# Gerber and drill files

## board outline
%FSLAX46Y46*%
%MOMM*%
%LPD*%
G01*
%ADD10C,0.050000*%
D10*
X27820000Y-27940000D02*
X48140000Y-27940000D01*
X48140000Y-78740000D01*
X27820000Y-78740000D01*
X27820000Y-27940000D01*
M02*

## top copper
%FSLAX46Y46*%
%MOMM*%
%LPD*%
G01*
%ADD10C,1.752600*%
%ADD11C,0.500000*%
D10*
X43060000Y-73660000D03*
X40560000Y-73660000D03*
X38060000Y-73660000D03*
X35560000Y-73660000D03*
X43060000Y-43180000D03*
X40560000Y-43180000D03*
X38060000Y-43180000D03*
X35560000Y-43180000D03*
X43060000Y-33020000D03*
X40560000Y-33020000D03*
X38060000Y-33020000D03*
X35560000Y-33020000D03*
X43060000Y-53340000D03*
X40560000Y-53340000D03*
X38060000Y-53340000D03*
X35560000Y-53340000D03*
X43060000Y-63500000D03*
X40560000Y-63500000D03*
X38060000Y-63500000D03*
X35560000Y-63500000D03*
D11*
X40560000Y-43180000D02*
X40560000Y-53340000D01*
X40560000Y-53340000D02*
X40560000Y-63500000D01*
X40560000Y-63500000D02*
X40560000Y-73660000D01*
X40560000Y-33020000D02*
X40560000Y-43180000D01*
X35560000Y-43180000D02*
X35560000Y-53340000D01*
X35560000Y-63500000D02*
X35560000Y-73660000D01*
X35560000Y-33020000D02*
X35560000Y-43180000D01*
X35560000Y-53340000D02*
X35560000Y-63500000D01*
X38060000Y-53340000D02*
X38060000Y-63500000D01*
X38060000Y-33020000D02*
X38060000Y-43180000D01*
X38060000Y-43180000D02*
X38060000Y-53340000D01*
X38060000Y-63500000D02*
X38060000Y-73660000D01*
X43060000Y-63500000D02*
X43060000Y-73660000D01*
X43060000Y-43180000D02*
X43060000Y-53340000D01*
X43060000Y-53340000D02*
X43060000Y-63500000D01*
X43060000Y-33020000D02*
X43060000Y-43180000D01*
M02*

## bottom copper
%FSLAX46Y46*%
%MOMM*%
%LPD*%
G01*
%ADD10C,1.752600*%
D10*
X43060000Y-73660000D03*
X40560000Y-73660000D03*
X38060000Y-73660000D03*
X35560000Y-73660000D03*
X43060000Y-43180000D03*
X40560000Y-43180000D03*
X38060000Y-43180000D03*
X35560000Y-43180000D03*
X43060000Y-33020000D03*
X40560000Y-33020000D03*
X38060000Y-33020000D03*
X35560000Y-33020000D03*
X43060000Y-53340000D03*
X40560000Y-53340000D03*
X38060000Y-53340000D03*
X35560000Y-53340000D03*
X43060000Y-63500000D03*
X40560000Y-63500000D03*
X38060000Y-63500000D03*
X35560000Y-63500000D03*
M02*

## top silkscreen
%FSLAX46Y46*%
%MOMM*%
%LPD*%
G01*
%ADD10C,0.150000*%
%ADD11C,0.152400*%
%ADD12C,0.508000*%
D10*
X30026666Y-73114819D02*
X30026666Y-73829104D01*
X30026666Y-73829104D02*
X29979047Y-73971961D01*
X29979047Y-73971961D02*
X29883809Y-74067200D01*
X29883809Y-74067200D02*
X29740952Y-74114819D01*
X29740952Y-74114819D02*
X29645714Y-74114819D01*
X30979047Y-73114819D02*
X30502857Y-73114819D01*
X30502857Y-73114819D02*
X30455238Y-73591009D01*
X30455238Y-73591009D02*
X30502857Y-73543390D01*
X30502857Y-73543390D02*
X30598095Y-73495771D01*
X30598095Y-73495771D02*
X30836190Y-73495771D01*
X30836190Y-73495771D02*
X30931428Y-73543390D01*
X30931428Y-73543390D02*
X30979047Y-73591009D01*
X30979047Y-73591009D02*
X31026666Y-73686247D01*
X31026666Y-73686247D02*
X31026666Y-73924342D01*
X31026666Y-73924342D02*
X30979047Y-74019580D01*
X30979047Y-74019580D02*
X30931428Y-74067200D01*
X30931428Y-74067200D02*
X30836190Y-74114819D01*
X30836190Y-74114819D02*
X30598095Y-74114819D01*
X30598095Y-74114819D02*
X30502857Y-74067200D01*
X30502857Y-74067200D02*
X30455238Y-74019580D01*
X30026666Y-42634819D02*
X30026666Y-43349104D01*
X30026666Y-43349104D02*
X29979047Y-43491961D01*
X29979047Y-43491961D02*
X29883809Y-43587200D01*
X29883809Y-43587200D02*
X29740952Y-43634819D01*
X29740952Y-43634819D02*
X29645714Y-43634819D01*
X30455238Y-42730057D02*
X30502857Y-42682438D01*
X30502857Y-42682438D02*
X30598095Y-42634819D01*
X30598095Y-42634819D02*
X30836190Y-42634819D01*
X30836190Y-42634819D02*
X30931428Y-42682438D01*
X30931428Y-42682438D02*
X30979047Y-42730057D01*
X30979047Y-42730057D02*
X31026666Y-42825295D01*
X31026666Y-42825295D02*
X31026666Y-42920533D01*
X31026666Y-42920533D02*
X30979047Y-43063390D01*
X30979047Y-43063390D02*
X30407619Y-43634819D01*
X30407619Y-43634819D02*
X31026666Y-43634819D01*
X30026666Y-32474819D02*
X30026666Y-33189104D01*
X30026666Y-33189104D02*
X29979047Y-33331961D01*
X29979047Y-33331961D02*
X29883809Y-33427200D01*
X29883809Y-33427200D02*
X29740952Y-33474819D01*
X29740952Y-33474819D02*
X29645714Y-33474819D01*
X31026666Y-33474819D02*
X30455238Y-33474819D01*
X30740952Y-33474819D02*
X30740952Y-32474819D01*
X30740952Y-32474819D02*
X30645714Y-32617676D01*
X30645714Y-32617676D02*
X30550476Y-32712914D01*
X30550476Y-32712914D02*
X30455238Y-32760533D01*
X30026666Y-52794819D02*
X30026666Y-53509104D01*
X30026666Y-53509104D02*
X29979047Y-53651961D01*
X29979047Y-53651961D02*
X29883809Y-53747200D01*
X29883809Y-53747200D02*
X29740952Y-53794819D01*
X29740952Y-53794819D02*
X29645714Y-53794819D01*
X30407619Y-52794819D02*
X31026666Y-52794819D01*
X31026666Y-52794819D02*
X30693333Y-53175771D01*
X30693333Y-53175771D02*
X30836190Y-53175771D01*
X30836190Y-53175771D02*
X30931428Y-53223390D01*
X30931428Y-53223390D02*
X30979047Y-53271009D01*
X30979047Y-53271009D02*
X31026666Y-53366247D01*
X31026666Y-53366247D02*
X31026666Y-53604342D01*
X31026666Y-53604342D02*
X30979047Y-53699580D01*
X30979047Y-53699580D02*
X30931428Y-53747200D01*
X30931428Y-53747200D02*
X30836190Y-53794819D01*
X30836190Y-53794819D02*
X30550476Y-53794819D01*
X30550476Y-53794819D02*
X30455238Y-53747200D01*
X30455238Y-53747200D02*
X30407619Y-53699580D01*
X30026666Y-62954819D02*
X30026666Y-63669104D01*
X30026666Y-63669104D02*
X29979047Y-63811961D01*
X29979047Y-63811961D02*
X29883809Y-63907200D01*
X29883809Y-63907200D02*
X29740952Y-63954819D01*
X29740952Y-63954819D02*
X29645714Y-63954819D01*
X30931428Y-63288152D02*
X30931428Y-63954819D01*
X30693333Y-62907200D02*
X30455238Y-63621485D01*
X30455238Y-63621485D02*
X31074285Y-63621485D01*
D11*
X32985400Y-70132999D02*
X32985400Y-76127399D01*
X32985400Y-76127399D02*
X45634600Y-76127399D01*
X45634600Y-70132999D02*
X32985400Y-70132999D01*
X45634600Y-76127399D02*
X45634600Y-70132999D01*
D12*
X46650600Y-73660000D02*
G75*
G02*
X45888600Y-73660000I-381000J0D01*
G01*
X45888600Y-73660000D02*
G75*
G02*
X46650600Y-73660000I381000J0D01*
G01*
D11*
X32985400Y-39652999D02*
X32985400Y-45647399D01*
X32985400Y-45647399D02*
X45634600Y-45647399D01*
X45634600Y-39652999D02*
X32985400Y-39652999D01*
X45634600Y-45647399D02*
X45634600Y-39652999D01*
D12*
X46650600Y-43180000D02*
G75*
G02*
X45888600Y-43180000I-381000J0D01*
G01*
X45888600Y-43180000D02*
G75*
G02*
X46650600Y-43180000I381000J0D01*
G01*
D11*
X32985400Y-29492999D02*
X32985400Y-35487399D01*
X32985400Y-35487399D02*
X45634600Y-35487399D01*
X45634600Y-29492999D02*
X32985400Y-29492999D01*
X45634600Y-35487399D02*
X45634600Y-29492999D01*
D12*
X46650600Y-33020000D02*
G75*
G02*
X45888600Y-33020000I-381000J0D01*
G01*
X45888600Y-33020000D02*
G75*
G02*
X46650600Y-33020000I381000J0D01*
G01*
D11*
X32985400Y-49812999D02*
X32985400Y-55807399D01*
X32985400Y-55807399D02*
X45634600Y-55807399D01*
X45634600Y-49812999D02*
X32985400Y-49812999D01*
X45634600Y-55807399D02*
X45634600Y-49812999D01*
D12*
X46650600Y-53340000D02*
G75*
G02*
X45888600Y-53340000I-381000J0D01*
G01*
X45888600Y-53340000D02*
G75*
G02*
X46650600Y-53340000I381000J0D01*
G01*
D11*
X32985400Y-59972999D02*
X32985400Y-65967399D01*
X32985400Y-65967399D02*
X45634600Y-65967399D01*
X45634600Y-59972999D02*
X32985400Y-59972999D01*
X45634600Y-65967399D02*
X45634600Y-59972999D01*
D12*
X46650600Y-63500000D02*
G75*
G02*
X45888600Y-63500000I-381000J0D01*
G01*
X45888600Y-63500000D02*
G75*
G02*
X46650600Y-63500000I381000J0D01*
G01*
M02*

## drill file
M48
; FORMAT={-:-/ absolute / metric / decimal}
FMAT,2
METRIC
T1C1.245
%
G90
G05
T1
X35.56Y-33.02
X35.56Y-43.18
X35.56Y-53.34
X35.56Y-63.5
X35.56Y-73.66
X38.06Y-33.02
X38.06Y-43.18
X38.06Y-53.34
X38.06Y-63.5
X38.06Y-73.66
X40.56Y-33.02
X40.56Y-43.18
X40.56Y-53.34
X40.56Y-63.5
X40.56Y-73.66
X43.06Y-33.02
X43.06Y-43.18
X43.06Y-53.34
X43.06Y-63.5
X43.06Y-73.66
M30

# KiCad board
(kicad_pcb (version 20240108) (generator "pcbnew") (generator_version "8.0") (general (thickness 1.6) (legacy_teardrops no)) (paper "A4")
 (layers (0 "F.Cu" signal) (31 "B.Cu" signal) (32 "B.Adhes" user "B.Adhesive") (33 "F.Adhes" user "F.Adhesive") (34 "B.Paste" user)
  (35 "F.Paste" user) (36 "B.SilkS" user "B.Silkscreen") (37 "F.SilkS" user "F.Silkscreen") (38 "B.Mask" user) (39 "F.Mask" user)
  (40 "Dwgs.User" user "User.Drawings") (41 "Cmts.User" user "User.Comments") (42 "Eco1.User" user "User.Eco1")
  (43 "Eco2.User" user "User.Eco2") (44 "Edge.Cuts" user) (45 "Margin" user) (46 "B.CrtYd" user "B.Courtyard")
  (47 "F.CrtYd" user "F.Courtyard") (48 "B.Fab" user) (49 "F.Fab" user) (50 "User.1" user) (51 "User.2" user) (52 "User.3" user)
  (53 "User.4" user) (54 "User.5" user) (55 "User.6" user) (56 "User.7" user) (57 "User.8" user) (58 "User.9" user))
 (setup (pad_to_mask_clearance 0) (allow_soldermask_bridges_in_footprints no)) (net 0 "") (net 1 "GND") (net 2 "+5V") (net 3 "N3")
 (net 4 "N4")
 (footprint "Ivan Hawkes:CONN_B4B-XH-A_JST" (layer "F.Cu") (at 43.06 73.66)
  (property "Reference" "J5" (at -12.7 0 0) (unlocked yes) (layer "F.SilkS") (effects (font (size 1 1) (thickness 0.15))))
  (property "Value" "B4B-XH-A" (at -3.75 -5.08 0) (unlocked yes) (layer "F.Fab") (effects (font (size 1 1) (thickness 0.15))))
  (fp_line (start -10.0746 -3.527001) (end -10.0746 2.467399) (stroke (width 0.1524) (type solid)) (layer "F.SilkS"))
  (fp_line (start -10.0746 2.467399) (end 2.5746 2.467399) (stroke (width 0.1524) (type solid)) (layer "F.SilkS"))
  (fp_line (start 2.5746 -3.527001) (end -10.0746 -3.527001) (stroke (width 0.1524) (type solid)) (layer "F.SilkS"))
  (fp_line (start 2.5746 2.467399) (end 2.5746 -3.527001) (stroke (width 0.1524) (type solid)) (layer "F.SilkS"))
  (fp_circle (center 3.2096 0) (end 3.5906 0) (stroke (width 0.508) (type solid)) (fill none) (layer "F.SilkS"))
  (pad "1" thru_hole circle (at 0 0) (size 1.7526 1.7526) (drill 1.2446) (layers "*.Cu" "*.Mask") (remove_unused_layers no) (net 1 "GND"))
  (pad "2" thru_hole circle (at -2.5 0) (size 1.7526 1.7526) (drill 1.2446) (layers "*.Cu" "*.Mask") (remove_unused_layers no) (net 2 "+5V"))
  (pad "3" thru_hole circle (at -5 0) (size 1.7526 1.7526) (drill 1.2446) (layers "*.Cu" "*.Mask") (remove_unused_layers no) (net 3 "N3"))
  (pad "4" thru_hole circle (at -7.5 0) (size 1.7526 1.7526) (drill 1.2446) (layers "*.Cu" "*.Mask") (remove_unused_layers no) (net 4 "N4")))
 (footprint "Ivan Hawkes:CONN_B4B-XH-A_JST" (layer "F.Cu") (at 43.06 43.18)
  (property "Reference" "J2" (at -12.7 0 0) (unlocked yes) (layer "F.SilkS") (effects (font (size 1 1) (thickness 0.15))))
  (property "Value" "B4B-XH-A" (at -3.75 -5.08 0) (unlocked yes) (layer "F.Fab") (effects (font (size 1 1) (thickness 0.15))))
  (fp_line (start -10.0746 -3.527001) (end -10.0746 2.467399) (stroke (width 0.1524) (type solid)) (layer "F.SilkS"))
  (fp_line (start -10.0746 2.467399) (end 2.5746 2.467399) (stroke (width 0.1524) (type solid)) (layer "F.SilkS"))
  (fp_line (start 2.5746 -3.527001) (end -10.0746 -3.527001) (stroke (width 0.1524) (type solid)) (layer "F.SilkS"))
  (fp_line (start 2.5746 2.467399) (end 2.5746 -3.527001) (stroke (width 0.1524) (type solid)) (layer "F.SilkS"))
  (fp_circle (center 3.2096 0) (end 3.5906 0) (stroke (width 0.508) (type solid)) (fill none) (layer "F.SilkS"))
  (pad "1" thru_hole circle (at 0 0) (size 1.7526 1.7526) (drill 1.2446) (layers "*.Cu" "*.Mask") (remove_unused_layers no) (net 1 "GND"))
  (pad "2" thru_hole circle (at -2.5 0) (size 1.7526 1.7526) (drill 1.2446) (layers "*.Cu" "*.Mask") (remove_unused_layers no) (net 2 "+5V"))
  (pad "3" thru_hole circle (at -5 0) (size 1.7526 1.7526) (drill 1.2446) (layers "*.Cu" "*.Mask") (remove_unused_layers no) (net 3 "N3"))
  (pad "4" thru_hole circle (at -7.5 0) (size 1.7526 1.7526) (drill 1.2446) (layers "*.Cu" "*.Mask") (remove_unused_layers no) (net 4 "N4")))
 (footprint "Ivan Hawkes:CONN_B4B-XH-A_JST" (layer "F.Cu") (at 43.06 33.02)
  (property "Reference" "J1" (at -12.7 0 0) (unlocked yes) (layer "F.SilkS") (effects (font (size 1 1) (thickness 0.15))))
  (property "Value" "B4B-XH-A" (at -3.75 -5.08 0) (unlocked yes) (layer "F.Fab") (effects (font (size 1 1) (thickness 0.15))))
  (fp_line (start -10.0746 -3.527001) (end -10.0746 2.467399) (stroke (width 0.1524) (type solid)) (layer "F.SilkS"))
  (fp_line (start -10.0746 2.467399) (end 2.5746 2.467399) (stroke (width 0.1524) (type solid)) (layer "F.SilkS"))
  (fp_line (start 2.5746 -3.527001) (end -10.0746 -3.527001) (stroke (width 0.1524) (type solid)) (layer "F.SilkS"))
  (fp_line (start 2.5746 2.467399) (end 2.5746 -3.527001) (stroke (width 0.1524) (type solid)) (layer "F.SilkS"))
  (fp_circle (center 3.2096 0) (end 3.5906 0) (stroke (width 0.508) (type solid)) (fill none) (layer "F.SilkS"))
  (pad "1" thru_hole circle (at 0 0) (size 1.7526 1.7526) (drill 1.2446) (layers "*.Cu" "*.Mask") (remove_unused_layers no) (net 1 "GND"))
  (pad "2" thru_hole circle (at -2.5 0) (size 1.7526 1.7526) (drill 1.2446) (layers "*.Cu" "*.Mask") (remove_unused_layers no) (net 2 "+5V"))
  (pad "3" thru_hole circle (at -5 0) (size 1.7526 1.7526) (drill 1.2446) (layers "*.Cu" "*.Mask") (remove_unused_layers no) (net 3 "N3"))
  (pad "4" thru_hole circle (at -7.5 0) (size 1.7526 1.7526) (drill 1.2446) (layers "*.Cu" "*.Mask") (remove_unused_layers no) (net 4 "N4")))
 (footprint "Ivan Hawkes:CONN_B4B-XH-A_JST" (layer "F.Cu") (at 43.06 53.34)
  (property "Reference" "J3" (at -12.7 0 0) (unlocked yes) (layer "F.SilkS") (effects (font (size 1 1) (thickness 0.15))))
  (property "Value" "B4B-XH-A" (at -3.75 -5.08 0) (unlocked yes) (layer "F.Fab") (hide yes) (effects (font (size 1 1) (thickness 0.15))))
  (fp_line (start -10.0746 -3.527001) (end -10.0746 2.467399) (stroke (width 0.1524) (type solid)) (layer "F.SilkS"))
  (fp_line (start -10.0746 2.467399) (end 2.5746 2.467399) (stroke (width 0.1524) (type solid)) (layer "F.SilkS"))
  (fp_line (start 2.5746 -3.527001) (end -10.0746 -3.527001) (stroke (width 0.1524) (type solid)) (layer "F.SilkS"))
  (fp_line (start 2.5746 2.467399) (end 2.5746 -3.527001) (stroke (width 0.1524) (type solid)) (layer "F.SilkS"))
  (fp_circle (center 3.2096 0) (end 3.5906 0) (stroke (width 0.508) (type solid)) (fill none) (layer "F.SilkS"))
  (pad "1" thru_hole circle (at 0 0) (size 1.7526 1.7526) (drill 1.2446) (layers "*.Cu" "*.Mask") (remove_unused_layers no) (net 1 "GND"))
  (pad "2" thru_hole circle (at -2.5 0) (size 1.7526 1.7526) (drill 1.2446) (layers "*.Cu" "*.Mask") (remove_unused_layers no) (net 2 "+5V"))
  (pad "3" thru_hole circle (at -5 0) (size 1.7526 1.7526) (drill 1.2446) (layers "*.Cu" "*.Mask") (remove_unused_layers no) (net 3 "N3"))
  (pad "4" thru_hole circle (at -7.5 0) (size 1.7526 1.7526) (drill 1.2446) (layers "*.Cu" "*.Mask") (remove_unused_layers no) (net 4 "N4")))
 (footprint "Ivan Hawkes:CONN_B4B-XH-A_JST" (layer "F.Cu") (at 43.06 63.5)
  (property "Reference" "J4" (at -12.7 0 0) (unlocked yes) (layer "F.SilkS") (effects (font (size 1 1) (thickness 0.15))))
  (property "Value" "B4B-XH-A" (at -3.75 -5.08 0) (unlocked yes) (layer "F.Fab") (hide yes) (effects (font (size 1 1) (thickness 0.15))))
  (fp_line (start -10.0746 -3.527001) (end -10.0746 2.467399) (stroke (width 0.1524) (type solid)) (layer "F.SilkS"))
  (fp_line (start -10.0746 2.467399) (end 2.5746 2.467399) (stroke (width 0.1524) (type solid)) (layer "F.SilkS"))
  (fp_line (start 2.5746 -3.527001) (end -10.0746 -3.527001) (stroke (width 0.1524) (type solid)) (layer "F.SilkS"))
  (fp_line (start 2.5746 2.467399) (end 2.5746 -3.527001) (stroke (width 0.1524) (type solid)) (layer "F.SilkS"))
  (fp_circle (center 3.2096 0) (end 3.5906 0) (stroke (width 0.508) (type solid)) (fill none) (layer "F.SilkS"))
  (pad "1" thru_hole circle (at 0 0) (size 1.7526 1.7526) (drill 1.2446) (layers "*.Cu" "*.Mask") (remove_unused_layers no) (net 1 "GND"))
  (pad "2" thru_hole circle (at -2.5 0) (size 1.7526 1.7526) (drill 1.2446) (layers "*.Cu" "*.Mask") (remove_unused_layers no) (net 2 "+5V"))
  (pad "3" thru_hole circle (at -5 0) (size 1.7526 1.7526) (drill 1.2446) (layers "*.Cu" "*.Mask") (remove_unused_layers no) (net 3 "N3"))
  (pad "4" thru_hole circle (at -7.5 0) (size 1.7526 1.7526) (drill 1.2446) (layers "*.Cu" "*.Mask") (remove_unused_layers no) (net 4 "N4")))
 (gr_rect (start 27.82 27.94) (end 48.14 78.74) (stroke (width 0.05) (type default)) (fill none) (layer "Edge.Cuts"))
 (segment (start 40.56 43.18) (end 40.56 53.34) (width 0.5) (layer "F.Cu") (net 2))
 (segment (start 40.56 53.34) (end 40.56 63.5) (width 0.5) (layer "F.Cu") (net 2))
 (segment (start 40.56 63.5) (end 40.56 73.66) (width 0.5) (layer "F.Cu") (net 2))
 (segment (start 40.56 33.02) (end 40.56 43.18) (width 0.5) (layer "F.Cu") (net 2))
 (segment (start 35.56 43.18) (end 35.56 53.34) (width 0.5) (layer "F.Cu") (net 4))
 (segment (start 35.56 63.5) (end 35.56 73.66) (width 0.5) (layer "F.Cu") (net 4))
 (segment (start 35.56 33.02) (end 35.56 43.18) (width 0.5) (layer "F.Cu") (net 4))
 (segment (start 35.56 53.34) (end 35.56 63.5) (width 0.5) (layer "F.Cu") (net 4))
 (segment (start 38.06 53.34) (end 38.06 63.5) (width 0.5) (layer "F.Cu") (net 3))
 (segment (start 38.06 33.02) (end 38.06 43.18) (width 0.5) (layer "F.Cu") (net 3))
 (segment (start 38.06 43.18) (end 38.06 53.34) (width 0.5) (layer "F.Cu") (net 3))
 (segment (start 38.06 63.5) (end 38.06 73.66) (width 0.5) (layer "F.Cu") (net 3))
 (segment (start 43.06 63.5) (end 43.06 73.66) (width 0.5) (layer "F.Cu") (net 1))
 (segment (start 43.06 43.18) (end 43.06 53.34) (width 0.5) (layer "F.Cu") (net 1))
 (segment (start 43.06 53.34) (end 43.06 63.5) (width 0.5) (layer "F.Cu") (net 1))
 (segment (start 43.06 33.02) (end 43.06 43.18) (width 0.5) (layer "F.Cu") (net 1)))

